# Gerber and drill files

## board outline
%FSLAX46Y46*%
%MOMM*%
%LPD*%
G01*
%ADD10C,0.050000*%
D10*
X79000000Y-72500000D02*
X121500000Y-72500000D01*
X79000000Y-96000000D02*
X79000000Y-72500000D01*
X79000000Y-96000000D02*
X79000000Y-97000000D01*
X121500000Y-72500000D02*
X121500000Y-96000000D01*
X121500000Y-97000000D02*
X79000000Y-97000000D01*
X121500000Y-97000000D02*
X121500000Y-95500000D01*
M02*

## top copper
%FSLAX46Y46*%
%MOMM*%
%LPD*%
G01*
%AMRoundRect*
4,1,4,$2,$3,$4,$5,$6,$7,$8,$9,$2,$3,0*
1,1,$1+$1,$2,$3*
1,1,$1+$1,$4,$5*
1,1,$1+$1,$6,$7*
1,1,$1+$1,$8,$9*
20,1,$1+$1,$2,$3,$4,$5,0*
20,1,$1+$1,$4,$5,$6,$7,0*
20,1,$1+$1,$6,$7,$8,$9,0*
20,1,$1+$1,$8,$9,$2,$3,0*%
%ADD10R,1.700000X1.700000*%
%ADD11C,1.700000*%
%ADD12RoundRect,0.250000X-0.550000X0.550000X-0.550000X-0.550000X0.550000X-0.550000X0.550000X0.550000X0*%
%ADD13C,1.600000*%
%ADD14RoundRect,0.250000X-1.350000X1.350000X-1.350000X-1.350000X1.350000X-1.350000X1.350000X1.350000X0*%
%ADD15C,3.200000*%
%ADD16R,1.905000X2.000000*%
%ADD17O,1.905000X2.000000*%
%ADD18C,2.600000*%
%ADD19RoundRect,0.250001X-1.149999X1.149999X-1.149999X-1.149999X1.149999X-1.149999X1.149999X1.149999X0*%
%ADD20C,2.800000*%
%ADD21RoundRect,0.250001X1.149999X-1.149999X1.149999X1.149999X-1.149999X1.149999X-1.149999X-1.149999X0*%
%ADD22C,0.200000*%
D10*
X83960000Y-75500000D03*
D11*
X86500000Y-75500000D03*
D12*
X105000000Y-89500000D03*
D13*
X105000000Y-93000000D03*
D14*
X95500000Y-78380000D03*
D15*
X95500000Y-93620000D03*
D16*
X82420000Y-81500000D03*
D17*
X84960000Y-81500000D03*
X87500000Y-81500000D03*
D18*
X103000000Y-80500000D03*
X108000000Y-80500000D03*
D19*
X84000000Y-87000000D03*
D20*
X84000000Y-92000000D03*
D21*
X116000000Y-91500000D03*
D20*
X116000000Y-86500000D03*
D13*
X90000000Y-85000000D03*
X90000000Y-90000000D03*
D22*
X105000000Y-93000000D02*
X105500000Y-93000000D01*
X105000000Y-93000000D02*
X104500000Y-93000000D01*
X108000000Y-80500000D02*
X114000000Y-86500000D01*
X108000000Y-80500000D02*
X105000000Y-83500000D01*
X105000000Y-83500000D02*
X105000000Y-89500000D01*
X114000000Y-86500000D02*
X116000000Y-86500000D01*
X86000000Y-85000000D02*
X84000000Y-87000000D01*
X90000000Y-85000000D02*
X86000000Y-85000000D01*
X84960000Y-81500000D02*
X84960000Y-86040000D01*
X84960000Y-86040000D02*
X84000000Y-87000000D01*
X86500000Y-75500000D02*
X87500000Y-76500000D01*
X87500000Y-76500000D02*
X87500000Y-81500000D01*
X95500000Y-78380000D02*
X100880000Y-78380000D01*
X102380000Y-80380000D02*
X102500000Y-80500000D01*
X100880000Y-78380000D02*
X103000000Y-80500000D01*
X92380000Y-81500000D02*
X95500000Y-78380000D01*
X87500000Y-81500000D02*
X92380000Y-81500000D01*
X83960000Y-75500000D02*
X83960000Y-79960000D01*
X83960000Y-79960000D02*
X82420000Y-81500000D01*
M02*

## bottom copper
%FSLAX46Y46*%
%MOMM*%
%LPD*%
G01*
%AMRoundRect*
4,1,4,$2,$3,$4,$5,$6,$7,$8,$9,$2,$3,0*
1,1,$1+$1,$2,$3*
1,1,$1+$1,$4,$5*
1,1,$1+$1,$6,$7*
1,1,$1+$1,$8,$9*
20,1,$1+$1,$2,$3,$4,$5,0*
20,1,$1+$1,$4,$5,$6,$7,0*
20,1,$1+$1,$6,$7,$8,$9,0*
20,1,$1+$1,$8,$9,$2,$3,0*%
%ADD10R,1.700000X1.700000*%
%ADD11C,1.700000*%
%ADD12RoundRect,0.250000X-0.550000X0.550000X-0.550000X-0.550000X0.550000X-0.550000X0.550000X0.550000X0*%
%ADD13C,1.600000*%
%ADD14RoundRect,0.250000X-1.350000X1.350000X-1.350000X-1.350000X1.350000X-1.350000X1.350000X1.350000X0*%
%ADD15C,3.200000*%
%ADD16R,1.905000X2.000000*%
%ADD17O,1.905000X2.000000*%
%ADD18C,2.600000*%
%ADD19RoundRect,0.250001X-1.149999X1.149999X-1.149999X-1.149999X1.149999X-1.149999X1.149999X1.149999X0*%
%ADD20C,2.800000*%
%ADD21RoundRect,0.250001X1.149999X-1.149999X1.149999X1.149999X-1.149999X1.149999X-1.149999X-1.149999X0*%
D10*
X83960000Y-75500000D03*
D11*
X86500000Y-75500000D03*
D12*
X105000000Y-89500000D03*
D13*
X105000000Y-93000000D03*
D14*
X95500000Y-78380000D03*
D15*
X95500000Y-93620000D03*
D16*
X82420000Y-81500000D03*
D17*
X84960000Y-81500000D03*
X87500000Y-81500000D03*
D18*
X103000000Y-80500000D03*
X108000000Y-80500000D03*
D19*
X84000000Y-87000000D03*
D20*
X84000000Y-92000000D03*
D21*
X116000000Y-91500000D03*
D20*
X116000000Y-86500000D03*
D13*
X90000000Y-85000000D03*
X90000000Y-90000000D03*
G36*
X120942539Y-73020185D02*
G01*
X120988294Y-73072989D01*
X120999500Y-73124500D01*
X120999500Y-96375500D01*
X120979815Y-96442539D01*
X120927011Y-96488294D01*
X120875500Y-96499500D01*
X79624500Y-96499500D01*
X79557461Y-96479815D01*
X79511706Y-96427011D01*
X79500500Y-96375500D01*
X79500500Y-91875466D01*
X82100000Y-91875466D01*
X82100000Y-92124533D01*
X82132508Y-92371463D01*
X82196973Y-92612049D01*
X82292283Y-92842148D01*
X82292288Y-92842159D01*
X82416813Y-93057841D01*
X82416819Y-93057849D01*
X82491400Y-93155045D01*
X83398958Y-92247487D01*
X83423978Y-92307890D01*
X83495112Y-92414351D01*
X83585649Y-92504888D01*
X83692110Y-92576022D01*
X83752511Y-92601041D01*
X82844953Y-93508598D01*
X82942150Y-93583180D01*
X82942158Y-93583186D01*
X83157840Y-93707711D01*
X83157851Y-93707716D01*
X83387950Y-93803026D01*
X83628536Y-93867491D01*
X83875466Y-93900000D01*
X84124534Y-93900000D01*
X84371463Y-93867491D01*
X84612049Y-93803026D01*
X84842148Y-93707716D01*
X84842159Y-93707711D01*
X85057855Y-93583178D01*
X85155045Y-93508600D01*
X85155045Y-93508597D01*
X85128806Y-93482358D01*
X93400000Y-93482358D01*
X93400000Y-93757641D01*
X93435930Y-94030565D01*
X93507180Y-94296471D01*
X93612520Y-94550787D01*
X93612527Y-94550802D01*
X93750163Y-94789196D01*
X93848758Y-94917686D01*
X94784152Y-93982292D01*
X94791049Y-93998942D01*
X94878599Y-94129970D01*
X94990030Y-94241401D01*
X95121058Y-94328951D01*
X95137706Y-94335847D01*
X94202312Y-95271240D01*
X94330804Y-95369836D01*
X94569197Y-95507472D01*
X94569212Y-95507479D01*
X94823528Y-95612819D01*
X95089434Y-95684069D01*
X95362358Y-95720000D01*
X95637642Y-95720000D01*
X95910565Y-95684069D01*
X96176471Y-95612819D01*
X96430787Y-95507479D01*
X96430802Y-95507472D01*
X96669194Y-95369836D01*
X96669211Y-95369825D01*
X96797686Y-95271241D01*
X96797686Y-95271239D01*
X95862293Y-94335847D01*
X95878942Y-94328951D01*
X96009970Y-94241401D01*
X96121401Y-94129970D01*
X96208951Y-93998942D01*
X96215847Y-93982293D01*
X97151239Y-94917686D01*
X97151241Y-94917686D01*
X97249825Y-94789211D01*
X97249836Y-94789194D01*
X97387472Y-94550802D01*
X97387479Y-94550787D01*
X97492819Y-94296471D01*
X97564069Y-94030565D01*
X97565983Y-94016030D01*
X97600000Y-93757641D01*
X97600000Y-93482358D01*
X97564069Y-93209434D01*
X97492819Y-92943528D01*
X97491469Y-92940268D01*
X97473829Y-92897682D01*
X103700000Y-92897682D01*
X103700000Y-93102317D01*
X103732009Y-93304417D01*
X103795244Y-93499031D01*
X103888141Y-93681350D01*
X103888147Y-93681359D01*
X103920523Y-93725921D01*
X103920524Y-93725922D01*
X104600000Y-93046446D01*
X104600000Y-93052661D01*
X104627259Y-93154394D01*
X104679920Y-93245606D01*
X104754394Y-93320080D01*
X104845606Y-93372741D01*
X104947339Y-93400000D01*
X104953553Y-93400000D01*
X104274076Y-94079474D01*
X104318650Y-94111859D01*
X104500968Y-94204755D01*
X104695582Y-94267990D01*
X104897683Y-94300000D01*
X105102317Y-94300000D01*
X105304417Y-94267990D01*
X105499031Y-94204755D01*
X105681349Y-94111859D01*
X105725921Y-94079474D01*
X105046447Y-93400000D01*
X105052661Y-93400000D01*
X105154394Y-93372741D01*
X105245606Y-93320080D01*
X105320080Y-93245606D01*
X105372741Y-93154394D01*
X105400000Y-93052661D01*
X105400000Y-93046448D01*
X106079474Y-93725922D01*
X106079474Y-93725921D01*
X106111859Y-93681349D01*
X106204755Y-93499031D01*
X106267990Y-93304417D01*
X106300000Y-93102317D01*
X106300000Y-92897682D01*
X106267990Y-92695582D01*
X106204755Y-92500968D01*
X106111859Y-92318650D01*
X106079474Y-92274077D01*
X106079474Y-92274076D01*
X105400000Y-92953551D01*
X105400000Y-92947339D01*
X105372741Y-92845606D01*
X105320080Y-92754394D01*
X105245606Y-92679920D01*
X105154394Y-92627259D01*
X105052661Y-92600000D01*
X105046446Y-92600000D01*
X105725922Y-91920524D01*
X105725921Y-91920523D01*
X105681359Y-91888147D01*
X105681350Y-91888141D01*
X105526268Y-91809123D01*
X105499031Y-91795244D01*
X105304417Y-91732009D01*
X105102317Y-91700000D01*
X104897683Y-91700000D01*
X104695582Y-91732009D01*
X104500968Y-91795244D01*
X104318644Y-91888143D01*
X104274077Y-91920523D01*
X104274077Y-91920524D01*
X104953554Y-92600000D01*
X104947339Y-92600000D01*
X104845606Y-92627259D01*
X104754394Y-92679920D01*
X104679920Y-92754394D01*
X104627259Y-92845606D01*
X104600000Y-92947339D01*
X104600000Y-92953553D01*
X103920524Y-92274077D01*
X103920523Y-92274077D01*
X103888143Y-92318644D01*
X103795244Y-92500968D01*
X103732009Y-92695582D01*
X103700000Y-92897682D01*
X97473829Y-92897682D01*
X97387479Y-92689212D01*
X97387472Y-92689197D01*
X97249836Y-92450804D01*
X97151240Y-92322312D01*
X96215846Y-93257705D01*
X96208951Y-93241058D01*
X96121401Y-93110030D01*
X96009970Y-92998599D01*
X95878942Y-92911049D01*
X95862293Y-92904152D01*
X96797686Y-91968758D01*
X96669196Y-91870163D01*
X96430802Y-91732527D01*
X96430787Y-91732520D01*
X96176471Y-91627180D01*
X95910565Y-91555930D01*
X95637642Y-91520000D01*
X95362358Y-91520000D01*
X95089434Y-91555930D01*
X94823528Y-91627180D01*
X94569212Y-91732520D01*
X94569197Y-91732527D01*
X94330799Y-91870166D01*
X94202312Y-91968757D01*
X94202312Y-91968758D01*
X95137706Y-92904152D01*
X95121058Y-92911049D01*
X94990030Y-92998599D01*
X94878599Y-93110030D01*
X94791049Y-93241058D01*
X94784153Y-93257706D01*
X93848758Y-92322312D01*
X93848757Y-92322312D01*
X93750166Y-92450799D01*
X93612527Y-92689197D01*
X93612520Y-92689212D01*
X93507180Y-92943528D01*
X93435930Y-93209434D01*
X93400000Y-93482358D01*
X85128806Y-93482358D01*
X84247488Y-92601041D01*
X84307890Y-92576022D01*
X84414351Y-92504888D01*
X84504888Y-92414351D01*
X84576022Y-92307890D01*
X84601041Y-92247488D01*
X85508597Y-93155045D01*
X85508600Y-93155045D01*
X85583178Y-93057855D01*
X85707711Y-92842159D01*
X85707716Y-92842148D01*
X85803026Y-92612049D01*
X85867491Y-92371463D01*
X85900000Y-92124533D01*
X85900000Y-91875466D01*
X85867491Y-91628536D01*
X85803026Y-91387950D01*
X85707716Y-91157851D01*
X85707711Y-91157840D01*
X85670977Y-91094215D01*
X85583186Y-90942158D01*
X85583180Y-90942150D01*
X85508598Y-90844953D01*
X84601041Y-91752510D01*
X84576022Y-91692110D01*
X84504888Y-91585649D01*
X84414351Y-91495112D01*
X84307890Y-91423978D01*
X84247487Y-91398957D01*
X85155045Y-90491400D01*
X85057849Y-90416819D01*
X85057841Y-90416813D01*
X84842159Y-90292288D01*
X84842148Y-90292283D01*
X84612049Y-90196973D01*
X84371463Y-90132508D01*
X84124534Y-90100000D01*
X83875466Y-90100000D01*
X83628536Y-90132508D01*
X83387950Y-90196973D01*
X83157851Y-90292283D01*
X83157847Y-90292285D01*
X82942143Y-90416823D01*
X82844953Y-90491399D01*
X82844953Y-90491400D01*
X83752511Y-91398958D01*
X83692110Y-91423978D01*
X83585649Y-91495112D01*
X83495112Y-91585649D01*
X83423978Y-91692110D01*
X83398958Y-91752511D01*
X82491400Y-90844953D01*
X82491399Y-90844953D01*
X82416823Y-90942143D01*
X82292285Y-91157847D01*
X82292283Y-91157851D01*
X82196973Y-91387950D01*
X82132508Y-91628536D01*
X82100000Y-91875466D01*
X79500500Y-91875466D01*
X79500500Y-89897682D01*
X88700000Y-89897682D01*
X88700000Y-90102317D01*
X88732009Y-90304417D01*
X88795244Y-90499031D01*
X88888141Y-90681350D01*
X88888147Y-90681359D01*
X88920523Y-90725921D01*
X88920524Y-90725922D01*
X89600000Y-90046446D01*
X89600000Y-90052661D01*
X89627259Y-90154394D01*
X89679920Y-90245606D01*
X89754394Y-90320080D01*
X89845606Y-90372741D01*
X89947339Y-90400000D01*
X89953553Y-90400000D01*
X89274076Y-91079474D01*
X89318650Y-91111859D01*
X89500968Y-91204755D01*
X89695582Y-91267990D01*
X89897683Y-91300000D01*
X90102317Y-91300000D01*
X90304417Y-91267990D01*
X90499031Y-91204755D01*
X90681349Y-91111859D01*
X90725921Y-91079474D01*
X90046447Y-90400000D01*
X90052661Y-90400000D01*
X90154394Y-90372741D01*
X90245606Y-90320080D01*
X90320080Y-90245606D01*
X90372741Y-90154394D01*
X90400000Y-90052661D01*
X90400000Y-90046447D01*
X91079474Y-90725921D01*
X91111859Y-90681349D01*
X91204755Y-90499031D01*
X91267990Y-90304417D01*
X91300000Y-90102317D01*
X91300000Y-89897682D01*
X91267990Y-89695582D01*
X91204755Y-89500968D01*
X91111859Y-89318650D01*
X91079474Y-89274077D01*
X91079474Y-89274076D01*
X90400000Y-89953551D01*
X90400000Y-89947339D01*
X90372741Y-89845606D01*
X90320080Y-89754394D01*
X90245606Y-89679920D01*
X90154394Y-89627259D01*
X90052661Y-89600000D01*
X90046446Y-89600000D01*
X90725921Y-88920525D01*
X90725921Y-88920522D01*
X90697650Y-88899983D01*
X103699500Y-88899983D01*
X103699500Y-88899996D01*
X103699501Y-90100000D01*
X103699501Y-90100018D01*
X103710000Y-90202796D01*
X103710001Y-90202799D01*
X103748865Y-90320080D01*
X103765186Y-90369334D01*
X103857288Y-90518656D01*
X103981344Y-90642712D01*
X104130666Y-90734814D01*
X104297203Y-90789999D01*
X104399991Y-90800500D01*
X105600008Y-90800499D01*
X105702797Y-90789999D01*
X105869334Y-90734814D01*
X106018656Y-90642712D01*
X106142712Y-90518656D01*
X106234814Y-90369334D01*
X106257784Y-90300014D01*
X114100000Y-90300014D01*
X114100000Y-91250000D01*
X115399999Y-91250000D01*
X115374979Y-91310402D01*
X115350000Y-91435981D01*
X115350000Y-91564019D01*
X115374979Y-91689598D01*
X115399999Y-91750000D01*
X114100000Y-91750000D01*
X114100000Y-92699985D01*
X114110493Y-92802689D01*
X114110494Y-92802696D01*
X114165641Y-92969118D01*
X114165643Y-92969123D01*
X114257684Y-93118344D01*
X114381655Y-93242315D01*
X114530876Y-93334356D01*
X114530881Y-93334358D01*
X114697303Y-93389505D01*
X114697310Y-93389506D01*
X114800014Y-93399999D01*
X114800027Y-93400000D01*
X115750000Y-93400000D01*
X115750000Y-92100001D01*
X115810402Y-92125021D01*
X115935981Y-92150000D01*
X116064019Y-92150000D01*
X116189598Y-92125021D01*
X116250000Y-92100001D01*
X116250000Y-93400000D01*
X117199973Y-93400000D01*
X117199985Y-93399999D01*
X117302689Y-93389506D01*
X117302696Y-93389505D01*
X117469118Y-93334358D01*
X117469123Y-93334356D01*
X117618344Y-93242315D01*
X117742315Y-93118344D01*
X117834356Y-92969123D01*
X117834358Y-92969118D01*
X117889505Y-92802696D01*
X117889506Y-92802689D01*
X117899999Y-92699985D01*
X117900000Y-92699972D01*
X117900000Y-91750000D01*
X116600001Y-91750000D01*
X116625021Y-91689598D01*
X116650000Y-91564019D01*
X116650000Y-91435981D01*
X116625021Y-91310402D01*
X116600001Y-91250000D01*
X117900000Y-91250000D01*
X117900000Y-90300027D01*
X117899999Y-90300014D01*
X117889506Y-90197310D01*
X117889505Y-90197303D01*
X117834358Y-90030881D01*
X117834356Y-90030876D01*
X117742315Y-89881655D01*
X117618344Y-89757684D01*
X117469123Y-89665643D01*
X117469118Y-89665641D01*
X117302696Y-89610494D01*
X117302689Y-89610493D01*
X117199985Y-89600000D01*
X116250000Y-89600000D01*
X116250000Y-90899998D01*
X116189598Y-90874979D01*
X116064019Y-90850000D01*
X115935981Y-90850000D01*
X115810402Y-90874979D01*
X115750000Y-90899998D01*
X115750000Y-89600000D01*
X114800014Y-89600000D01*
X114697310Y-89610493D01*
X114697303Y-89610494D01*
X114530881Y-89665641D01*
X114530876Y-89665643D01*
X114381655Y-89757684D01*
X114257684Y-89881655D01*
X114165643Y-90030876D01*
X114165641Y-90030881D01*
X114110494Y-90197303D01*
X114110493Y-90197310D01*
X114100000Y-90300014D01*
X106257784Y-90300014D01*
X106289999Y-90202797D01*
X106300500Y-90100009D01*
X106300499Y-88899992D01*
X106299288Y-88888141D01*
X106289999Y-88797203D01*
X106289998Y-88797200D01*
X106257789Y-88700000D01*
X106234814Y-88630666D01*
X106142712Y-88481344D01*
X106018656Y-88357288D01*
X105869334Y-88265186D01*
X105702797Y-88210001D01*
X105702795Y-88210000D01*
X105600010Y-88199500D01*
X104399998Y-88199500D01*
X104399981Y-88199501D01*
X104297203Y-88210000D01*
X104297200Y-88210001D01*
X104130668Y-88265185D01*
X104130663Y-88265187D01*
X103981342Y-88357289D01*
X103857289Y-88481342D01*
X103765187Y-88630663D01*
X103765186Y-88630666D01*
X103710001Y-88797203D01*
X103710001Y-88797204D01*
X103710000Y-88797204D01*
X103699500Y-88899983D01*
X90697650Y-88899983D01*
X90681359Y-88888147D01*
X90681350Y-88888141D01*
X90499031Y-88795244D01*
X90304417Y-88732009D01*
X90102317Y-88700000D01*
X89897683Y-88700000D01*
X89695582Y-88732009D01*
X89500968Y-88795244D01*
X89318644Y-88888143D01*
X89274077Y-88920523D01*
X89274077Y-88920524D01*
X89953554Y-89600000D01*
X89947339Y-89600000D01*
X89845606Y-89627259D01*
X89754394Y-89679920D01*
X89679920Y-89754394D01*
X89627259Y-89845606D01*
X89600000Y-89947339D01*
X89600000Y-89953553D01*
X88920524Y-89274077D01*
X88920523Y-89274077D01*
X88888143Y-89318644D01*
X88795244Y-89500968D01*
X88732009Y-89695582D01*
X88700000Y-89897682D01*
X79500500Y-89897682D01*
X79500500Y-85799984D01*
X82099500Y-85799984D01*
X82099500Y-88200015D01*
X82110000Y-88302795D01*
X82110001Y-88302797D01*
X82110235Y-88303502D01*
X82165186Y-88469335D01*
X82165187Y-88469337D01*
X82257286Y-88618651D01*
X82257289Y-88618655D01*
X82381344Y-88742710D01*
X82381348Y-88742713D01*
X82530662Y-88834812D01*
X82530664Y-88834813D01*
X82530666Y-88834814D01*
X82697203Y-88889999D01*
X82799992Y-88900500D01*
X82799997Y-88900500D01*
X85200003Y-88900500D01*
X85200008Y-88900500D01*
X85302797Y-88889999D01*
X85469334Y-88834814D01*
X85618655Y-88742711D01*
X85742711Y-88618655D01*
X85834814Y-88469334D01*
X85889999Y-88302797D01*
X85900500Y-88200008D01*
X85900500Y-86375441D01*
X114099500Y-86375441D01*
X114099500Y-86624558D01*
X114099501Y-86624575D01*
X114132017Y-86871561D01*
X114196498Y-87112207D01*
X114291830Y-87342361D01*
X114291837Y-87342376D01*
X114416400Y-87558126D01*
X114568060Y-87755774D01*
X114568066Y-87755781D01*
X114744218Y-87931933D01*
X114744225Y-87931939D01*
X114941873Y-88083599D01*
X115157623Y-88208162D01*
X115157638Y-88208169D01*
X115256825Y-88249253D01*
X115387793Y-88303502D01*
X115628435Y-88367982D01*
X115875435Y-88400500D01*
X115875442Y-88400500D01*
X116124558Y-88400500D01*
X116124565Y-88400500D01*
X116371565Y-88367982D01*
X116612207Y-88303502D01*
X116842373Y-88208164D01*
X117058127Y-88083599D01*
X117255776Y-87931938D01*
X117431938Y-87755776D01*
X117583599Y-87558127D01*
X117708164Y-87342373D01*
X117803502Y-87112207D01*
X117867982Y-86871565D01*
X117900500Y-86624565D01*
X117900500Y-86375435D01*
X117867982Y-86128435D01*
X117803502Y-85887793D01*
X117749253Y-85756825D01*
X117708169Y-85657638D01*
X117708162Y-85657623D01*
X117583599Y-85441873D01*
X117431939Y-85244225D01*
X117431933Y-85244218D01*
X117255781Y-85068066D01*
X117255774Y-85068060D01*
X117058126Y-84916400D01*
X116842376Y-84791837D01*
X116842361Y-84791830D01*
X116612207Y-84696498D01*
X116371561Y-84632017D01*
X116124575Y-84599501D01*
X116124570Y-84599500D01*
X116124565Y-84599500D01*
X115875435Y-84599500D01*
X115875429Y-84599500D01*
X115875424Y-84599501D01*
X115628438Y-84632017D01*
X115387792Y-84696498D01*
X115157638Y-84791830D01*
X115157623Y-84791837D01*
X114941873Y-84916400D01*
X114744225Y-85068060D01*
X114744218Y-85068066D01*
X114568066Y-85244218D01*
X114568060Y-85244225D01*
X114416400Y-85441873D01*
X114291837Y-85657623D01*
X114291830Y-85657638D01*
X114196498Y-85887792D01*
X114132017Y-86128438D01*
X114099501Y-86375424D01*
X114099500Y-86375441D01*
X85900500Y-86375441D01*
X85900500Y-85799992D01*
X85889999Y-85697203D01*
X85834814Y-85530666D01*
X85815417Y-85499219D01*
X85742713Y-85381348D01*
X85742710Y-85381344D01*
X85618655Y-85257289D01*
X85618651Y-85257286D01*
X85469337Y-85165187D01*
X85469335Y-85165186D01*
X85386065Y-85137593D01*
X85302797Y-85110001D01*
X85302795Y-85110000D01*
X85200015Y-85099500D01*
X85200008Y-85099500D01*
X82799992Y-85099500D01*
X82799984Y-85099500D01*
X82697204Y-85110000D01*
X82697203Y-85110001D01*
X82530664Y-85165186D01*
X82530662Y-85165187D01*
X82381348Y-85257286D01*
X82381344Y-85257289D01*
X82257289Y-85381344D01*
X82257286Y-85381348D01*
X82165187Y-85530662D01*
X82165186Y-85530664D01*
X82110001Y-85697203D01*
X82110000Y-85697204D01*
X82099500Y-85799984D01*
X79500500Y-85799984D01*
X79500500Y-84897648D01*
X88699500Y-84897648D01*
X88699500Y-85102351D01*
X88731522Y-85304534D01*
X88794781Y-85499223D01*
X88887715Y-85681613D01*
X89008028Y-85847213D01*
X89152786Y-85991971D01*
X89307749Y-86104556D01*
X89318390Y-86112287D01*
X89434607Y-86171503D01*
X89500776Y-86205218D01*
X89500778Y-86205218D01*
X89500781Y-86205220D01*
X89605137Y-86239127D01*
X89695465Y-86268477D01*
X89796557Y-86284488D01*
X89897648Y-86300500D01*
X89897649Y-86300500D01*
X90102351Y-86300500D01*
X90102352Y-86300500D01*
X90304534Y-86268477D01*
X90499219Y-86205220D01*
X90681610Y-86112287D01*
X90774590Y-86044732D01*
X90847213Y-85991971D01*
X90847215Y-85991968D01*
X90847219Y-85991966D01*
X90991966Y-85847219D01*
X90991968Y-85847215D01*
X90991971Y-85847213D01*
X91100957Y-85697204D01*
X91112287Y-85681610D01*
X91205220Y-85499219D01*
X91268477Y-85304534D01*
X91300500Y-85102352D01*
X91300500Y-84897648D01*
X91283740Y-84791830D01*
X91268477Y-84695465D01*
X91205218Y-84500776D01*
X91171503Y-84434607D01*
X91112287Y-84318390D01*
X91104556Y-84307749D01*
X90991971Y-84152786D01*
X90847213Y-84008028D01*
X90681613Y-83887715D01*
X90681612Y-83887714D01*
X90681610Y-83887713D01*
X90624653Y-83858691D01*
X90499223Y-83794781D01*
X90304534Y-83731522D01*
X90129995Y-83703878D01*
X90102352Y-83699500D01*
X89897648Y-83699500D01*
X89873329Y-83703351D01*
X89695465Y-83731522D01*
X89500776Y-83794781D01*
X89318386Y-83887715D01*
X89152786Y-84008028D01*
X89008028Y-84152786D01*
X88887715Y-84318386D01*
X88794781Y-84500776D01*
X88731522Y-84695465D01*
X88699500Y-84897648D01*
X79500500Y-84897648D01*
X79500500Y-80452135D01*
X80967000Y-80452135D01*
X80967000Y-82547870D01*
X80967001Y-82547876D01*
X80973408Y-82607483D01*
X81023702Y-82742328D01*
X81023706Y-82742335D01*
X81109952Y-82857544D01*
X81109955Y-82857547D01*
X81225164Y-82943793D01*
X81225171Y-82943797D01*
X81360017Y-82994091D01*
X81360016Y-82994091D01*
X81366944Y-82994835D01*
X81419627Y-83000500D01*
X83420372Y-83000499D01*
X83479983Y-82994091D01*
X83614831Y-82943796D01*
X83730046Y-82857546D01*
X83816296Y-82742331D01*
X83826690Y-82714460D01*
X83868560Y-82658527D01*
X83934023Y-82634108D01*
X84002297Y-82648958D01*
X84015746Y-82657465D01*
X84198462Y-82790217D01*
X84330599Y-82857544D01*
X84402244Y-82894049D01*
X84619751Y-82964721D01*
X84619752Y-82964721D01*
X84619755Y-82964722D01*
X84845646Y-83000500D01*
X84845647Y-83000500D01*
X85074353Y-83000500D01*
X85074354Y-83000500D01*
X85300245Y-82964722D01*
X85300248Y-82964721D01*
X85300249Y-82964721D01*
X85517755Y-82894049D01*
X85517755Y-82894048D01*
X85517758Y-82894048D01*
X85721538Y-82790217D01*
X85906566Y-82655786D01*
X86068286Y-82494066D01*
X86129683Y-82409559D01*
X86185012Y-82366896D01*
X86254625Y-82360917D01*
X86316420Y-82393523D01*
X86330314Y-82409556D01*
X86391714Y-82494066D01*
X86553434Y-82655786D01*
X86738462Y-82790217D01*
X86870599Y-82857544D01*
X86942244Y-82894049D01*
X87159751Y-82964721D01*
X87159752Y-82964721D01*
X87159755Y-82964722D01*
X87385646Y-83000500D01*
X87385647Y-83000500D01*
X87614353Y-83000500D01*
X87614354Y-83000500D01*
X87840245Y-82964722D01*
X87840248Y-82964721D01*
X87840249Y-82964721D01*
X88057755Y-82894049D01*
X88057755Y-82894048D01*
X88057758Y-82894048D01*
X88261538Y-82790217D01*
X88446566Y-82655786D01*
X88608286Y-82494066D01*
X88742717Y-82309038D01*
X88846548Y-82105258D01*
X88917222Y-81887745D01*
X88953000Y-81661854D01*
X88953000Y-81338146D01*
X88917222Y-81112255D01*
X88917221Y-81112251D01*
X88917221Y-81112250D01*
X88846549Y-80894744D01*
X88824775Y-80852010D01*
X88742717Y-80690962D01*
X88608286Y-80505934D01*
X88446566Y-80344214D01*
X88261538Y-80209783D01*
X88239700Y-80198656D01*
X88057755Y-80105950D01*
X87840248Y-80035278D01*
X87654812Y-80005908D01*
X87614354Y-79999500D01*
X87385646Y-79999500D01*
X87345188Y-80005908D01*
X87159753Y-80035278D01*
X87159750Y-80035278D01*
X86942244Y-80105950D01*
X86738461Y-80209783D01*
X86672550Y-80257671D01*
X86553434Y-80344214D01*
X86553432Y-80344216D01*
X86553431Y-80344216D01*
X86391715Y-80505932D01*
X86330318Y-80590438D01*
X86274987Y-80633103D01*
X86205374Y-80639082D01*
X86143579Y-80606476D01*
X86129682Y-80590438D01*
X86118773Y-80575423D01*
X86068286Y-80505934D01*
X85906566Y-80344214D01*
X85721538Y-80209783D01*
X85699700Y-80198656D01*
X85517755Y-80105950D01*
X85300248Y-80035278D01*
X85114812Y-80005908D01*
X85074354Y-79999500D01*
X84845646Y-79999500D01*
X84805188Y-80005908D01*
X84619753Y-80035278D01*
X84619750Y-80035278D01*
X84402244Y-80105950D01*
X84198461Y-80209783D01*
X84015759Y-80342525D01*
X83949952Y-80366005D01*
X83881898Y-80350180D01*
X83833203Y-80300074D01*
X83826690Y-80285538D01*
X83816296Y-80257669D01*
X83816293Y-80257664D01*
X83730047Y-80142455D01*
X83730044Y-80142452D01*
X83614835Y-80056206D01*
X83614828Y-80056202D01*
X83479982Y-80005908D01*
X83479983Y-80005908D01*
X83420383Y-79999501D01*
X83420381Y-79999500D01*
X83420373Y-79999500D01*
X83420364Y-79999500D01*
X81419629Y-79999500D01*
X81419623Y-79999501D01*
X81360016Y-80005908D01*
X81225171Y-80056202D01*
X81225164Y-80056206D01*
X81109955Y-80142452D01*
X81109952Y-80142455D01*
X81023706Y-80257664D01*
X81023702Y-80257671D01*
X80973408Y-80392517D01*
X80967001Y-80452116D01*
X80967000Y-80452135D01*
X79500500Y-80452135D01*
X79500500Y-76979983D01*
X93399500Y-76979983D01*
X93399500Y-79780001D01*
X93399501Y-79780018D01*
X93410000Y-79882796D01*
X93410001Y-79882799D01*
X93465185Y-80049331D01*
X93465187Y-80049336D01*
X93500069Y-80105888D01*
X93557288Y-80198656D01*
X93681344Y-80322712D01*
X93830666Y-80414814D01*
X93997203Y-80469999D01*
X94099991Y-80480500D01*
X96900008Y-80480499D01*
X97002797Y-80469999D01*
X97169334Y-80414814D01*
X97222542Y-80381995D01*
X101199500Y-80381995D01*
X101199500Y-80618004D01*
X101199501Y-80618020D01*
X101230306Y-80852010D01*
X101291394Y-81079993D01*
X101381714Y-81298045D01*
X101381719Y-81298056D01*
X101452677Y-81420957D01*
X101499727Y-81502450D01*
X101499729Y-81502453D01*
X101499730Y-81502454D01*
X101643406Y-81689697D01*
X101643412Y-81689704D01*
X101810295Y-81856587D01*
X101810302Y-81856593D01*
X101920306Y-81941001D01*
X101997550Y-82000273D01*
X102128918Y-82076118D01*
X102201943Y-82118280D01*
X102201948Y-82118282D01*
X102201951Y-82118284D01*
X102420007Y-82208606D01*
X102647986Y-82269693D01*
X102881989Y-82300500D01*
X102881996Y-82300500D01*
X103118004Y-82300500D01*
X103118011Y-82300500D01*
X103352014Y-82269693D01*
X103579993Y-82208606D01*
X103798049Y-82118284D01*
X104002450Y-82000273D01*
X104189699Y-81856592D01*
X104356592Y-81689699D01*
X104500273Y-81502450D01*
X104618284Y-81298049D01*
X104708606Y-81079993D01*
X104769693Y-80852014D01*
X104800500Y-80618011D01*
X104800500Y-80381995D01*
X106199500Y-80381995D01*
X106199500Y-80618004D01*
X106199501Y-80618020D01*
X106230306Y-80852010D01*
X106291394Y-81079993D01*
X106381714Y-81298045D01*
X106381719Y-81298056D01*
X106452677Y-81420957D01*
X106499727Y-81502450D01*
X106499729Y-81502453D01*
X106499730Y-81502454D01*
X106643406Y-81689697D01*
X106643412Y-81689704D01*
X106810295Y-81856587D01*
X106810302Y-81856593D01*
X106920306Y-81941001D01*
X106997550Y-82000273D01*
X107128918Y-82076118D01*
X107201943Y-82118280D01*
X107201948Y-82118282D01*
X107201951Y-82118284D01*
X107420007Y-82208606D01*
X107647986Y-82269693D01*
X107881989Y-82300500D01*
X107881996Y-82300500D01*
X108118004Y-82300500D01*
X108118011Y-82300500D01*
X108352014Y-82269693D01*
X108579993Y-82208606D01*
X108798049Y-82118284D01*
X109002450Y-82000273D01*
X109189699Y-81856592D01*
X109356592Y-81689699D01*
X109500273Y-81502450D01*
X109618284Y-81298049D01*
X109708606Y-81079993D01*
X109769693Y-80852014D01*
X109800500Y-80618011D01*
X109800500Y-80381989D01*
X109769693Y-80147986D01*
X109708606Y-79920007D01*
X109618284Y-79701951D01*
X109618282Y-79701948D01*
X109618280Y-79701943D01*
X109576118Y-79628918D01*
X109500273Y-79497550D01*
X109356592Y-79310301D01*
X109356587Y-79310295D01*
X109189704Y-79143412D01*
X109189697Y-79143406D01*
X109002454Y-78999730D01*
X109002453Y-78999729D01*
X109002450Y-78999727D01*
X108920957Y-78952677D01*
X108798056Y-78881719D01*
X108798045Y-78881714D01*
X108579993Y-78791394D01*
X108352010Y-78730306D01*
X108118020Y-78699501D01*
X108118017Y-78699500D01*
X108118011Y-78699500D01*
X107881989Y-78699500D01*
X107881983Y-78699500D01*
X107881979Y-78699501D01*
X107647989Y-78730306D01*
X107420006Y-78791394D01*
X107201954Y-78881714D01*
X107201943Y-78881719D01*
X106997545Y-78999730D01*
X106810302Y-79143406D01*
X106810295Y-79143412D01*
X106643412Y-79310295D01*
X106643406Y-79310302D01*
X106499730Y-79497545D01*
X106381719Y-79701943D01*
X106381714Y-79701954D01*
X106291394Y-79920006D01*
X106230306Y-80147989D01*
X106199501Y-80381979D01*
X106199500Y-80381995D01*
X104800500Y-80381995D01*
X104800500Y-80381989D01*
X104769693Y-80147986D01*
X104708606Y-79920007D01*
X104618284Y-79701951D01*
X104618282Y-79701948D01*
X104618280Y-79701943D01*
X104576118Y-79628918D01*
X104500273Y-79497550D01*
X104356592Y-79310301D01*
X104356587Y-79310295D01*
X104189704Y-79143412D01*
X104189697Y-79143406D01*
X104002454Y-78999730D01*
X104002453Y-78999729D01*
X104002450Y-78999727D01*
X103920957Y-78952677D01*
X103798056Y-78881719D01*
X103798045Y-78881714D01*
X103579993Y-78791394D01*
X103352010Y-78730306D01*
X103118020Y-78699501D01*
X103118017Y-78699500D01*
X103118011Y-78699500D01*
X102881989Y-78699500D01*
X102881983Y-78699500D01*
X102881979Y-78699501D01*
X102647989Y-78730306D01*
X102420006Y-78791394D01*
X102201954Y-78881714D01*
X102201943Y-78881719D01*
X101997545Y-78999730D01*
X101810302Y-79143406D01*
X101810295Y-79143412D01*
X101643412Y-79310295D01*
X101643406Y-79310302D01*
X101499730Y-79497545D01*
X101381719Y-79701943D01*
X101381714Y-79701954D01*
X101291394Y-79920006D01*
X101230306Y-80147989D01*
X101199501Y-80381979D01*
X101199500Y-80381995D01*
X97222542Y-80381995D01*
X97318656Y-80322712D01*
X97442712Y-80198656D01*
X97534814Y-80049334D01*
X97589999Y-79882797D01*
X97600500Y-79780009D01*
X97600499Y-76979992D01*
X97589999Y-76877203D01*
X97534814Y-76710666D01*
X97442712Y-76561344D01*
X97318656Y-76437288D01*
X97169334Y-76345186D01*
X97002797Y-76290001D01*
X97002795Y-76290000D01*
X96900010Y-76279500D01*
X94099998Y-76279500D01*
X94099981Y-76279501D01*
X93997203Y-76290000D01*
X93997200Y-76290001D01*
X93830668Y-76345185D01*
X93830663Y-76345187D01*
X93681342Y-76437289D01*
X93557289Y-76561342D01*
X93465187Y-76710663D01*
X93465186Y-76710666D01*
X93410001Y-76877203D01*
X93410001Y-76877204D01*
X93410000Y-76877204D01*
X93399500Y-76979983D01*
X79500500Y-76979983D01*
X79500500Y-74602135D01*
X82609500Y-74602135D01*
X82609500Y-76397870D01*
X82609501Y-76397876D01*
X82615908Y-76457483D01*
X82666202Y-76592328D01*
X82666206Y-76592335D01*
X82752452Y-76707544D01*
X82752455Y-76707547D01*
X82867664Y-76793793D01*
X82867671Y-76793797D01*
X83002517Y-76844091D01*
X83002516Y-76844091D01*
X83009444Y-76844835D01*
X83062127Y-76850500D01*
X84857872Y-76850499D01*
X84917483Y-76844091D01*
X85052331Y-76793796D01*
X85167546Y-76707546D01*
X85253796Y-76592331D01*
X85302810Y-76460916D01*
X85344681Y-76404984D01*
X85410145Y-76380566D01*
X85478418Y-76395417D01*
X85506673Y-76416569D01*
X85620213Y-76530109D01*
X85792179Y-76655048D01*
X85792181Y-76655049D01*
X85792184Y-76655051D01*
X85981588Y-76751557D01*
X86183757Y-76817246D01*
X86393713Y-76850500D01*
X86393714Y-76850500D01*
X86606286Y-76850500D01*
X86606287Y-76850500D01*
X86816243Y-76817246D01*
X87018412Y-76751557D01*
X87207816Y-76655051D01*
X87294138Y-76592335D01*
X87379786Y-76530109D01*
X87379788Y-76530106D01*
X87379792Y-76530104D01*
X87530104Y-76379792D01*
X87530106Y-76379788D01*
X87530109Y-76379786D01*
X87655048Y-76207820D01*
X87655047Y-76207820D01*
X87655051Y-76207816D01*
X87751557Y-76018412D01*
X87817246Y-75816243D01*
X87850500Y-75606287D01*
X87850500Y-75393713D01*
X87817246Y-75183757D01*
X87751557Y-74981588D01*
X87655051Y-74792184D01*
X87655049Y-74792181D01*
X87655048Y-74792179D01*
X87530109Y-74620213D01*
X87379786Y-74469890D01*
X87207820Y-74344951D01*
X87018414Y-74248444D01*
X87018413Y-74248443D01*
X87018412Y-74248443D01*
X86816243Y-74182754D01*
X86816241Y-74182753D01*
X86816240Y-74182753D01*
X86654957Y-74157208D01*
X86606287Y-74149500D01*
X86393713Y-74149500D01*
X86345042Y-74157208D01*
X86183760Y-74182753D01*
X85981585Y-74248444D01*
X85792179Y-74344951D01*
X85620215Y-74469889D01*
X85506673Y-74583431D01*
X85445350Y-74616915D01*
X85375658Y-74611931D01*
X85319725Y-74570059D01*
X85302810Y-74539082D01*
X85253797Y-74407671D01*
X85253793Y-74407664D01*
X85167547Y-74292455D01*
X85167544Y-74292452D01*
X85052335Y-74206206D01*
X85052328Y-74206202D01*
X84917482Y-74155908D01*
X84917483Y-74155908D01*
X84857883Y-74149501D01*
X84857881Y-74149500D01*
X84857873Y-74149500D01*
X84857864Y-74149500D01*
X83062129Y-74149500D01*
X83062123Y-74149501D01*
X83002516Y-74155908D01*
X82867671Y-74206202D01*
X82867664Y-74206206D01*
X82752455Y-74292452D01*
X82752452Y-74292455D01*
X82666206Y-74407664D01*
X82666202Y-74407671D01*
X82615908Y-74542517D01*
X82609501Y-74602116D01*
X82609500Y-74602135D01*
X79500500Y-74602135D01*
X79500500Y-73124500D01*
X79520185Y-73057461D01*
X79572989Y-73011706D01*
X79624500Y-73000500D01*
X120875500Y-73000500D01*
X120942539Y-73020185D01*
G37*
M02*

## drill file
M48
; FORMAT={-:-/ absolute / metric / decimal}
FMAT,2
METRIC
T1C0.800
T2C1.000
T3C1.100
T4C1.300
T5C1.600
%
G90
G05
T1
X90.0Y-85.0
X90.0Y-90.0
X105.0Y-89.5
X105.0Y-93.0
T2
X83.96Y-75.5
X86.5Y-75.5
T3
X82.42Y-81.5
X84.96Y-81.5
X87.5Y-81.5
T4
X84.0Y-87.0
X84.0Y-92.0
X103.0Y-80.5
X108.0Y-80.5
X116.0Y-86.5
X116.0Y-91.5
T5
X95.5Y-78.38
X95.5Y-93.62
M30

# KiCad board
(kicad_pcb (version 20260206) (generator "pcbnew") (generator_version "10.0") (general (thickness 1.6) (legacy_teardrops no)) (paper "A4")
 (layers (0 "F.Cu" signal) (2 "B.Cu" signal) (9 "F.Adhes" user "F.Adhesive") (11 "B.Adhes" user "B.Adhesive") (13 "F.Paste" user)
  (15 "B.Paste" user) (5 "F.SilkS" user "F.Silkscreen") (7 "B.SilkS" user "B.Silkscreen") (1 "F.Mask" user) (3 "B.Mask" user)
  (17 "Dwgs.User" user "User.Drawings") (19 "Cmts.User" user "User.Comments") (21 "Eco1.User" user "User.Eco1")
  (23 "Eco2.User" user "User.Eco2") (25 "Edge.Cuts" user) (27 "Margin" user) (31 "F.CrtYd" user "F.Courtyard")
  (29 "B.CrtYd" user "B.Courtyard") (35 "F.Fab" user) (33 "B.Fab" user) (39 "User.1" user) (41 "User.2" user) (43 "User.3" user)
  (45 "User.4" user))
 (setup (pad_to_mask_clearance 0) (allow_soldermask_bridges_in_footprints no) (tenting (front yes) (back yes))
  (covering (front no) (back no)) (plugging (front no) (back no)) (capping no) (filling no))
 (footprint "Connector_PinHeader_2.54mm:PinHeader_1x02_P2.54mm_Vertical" (layer "F.Cu") (at 83.96 75.5 90)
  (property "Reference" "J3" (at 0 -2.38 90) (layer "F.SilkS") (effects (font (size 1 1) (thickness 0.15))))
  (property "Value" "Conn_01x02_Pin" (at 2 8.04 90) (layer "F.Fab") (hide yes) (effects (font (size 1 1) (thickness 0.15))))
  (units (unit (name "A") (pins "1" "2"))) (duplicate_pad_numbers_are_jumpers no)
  (pad "1" thru_hole rect (at 0 0 90) (size 1.7 1.7) (drill 1) (layers "*.Cu" "*.Mask") (remove_unused_layers no) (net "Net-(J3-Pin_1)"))
  (pad "2" thru_hole circle (at 0 2.54 90) (size 1.7 1.7) (drill 1) (layers "*.Cu" "*.Mask") (remove_unused_layers no) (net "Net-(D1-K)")))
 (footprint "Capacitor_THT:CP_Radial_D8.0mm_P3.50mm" (layer "F.Cu") (at 105 89.5 -90)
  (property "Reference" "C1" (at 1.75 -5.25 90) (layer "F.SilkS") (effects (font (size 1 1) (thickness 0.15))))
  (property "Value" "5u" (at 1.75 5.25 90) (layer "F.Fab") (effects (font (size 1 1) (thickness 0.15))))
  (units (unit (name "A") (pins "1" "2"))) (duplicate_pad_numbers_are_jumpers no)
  (pad "1" thru_hole roundrect (at 0 0 270) (size 1.6 1.6) (drill 0.8) (layers "*.Cu" "*.Mask") (remove_unused_layers no)
   (roundrect_rratio 0.15625) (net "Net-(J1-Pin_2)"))
  (pad "2" thru_hole circle (at 3.5 0 270) (size 1.6 1.6) (drill 0.8) (layers "*.Cu" "*.Mask") (remove_unused_layers no) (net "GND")))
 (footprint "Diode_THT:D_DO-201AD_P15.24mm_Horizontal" (layer "F.Cu") (at 95.5 78.38 -90)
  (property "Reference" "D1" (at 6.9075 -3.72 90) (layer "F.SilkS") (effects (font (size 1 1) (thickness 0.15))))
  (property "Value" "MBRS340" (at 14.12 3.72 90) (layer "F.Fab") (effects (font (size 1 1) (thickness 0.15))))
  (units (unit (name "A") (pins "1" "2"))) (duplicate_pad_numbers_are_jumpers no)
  (pad "1" thru_hole roundrect (at 0 0 270) (size 3.2 3.2) (drill 1.6) (layers "*.Cu" "*.Mask") (remove_unused_layers no)
   (roundrect_rratio 0.078125) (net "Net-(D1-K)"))
  (pad "2" thru_hole circle (at 15.24 0 270) (size 3.2 3.2) (drill 1.6) (layers "*.Cu" "*.Mask") (remove_unused_layers no) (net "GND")))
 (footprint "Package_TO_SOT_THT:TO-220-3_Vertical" (layer "F.Cu") (at 82.42 81.5)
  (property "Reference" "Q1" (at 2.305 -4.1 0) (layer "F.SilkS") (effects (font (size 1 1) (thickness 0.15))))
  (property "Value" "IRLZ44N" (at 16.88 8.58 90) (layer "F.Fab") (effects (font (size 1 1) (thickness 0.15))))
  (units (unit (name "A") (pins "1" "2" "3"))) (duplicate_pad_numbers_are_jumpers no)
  (pad "1" thru_hole rect (at 0 0) (size 1.905 2) (drill 1.1) (layers "*.Cu" "*.Mask") (remove_unused_layers no) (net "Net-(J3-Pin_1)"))
  (pad "2" thru_hole oval (at 2.54 0) (size 1.905 2) (drill 1.1) (layers "*.Cu" "*.Mask") (remove_unused_layers no) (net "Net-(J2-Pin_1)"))
  (pad "3" thru_hole oval (at 5.08 0) (size 1.905 2) (drill 1.1) (layers "*.Cu" "*.Mask") (remove_unused_layers no) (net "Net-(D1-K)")))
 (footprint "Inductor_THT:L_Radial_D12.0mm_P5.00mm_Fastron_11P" (layer "F.Cu") (at 103 80.5)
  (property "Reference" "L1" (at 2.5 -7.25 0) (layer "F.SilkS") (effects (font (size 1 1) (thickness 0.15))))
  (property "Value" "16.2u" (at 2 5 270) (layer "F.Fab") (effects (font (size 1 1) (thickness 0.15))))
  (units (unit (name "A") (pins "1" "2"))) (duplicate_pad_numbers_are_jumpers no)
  (pad "1" thru_hole circle (at 0 0) (size 2.6 2.6) (drill 1.3) (layers "*.Cu" "*.Mask") (remove_unused_layers no) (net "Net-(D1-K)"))
  (pad "2" thru_hole circle (at 5 0) (size 2.6 2.6) (drill 1.3) (layers "*.Cu" "*.Mask") (remove_unused_layers no) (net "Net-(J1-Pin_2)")))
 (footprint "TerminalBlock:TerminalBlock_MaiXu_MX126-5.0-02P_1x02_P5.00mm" (layer "F.Cu") (at 84 87 -90)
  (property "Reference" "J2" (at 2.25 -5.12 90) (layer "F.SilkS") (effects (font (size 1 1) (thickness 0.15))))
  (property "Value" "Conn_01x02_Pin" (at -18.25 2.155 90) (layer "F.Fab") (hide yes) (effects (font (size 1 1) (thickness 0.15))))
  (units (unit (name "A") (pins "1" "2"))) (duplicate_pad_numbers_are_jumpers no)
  (pad "1" thru_hole roundrect (at 0 0 270) (size 2.8 2.8) (drill 1.3) (layers "*.Cu" "*.Mask") (remove_unused_layers no)
   (roundrect_rratio 0.089286) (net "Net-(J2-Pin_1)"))
  (pad "2" thru_hole circle (at 5 0 270) (size 2.8 2.8) (drill 1.3) (layers "*.Cu" "*.Mask") (remove_unused_layers no) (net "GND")))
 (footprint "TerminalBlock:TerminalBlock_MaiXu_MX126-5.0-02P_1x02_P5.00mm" (layer "F.Cu") (at 116 91.5 90)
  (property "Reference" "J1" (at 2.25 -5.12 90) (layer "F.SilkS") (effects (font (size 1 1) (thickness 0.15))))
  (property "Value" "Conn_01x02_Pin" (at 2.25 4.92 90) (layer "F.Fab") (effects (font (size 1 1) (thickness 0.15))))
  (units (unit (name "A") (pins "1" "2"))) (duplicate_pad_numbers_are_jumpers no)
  (pad "1" thru_hole roundrect (at 0 0 90) (size 2.8 2.8) (drill 1.3) (layers "*.Cu" "*.Mask") (remove_unused_layers no)
   (roundrect_rratio 0.089286) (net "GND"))
  (pad "2" thru_hole circle (at 5 0 90) (size 2.8 2.8) (drill 1.3) (layers "*.Cu" "*.Mask") (remove_unused_layers no) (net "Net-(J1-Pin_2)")))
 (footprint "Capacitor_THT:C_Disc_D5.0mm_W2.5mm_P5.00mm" (layer "F.Cu") (at 90 85 -90)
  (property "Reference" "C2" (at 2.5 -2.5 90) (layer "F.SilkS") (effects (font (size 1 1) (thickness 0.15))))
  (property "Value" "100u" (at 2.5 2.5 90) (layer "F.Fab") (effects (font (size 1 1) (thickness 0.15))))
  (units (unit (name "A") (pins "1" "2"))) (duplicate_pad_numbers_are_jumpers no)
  (pad "1" thru_hole circle (at 0 0 270) (size 1.6 1.6) (drill 0.8) (layers "*.Cu" "*.Mask") (remove_unused_layers no)
   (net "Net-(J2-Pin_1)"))
  (pad "2" thru_hole circle (at 5 0 270) (size 1.6 1.6) (drill 0.8) (layers "*.Cu" "*.Mask") (remove_unused_layers no) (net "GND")))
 (gr_line (start 79 72.5) (end 121.5 72.5) (stroke (width 0.05) (type default)) (layer "Edge.Cuts"))
 (gr_line (start 79 96) (end 79 72.5) (stroke (width 0.05) (type default)) (layer "Edge.Cuts"))
 (gr_line (start 79 96) (end 79 97) (stroke (width 0.05) (type default)) (layer "Edge.Cuts"))
 (gr_line (start 121.5 72.5) (end 121.5 96) (stroke (width 0.05) (type default)) (layer "Edge.Cuts"))
 (gr_line (start 121.5 97) (end 79 97) (stroke (width 0.05) (type default)) (layer "Edge.Cuts"))
 (gr_line (start 121.5 97) (end 121.5 95.5) (stroke (width 0.05) (type default)) (layer "Edge.Cuts"))
 (segment (start 105 93) (end 105.5 93) (width 0.2) (layer "F.Cu") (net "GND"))
 (segment (start 105 93) (end 104.5 93) (width 0.2) (layer "F.Cu") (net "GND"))
 (segment (start 108 80.5) (end 114 86.5) (width 0.2) (layer "F.Cu") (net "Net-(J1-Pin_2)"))
 (segment (start 108 80.5) (end 105 83.5) (width 0.2) (layer "F.Cu") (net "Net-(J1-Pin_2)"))
 (segment (start 105 83.5) (end 105 89.5) (width 0.2) (layer "F.Cu") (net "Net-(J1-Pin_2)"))
 (segment (start 114 86.5) (end 116 86.5) (width 0.2) (layer "F.Cu") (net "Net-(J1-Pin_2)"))
 (segment (start 86 85) (end 84 87) (width 0.2) (layer "F.Cu") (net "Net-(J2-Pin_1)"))
 (segment (start 90 85) (end 86 85) (width 0.2) (layer "F.Cu") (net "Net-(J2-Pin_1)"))
 (segment (start 84.96 81.5) (end 84.96 86.04) (width 0.2) (layer "F.Cu") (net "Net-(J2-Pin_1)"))
 (segment (start 84.96 86.04) (end 84 87) (width 0.2) (layer "F.Cu") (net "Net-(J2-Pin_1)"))
 (segment (start 86.5 75.5) (end 87.5 76.5) (width 0.2) (layer "F.Cu") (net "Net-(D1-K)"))
 (segment (start 87.5 76.5) (end 87.5 81.5) (width 0.2) (layer "F.Cu") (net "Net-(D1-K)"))
 (segment (start 95.5 78.38) (end 100.88 78.38) (width 0.2) (layer "F.Cu") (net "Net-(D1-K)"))
 (segment (start 102.38 80.38) (end 102.5 80.5) (width 0.2) (layer "F.Cu") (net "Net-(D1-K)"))
 (segment (start 100.88 78.38) (end 103 80.5) (width 0.2) (layer "F.Cu") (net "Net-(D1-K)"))
 (segment (start 92.38 81.5) (end 95.5 78.38) (width 0.2) (layer "F.Cu") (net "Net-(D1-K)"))
 (segment (start 87.5 81.5) (end 92.38 81.5) (width 0.2) (layer "F.Cu") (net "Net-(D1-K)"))
 (segment (start 83.96 75.5) (end 83.96 79.96) (width 0.2) (layer "F.Cu") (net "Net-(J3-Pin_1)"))
 (segment (start 83.96 79.96) (end 82.42 81.5) (width 0.2) (layer "F.Cu") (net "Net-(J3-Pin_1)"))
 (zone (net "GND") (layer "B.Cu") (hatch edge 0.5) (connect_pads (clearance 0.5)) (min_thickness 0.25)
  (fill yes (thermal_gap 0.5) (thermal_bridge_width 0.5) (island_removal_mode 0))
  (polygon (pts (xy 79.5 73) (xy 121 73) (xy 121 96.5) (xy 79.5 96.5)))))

